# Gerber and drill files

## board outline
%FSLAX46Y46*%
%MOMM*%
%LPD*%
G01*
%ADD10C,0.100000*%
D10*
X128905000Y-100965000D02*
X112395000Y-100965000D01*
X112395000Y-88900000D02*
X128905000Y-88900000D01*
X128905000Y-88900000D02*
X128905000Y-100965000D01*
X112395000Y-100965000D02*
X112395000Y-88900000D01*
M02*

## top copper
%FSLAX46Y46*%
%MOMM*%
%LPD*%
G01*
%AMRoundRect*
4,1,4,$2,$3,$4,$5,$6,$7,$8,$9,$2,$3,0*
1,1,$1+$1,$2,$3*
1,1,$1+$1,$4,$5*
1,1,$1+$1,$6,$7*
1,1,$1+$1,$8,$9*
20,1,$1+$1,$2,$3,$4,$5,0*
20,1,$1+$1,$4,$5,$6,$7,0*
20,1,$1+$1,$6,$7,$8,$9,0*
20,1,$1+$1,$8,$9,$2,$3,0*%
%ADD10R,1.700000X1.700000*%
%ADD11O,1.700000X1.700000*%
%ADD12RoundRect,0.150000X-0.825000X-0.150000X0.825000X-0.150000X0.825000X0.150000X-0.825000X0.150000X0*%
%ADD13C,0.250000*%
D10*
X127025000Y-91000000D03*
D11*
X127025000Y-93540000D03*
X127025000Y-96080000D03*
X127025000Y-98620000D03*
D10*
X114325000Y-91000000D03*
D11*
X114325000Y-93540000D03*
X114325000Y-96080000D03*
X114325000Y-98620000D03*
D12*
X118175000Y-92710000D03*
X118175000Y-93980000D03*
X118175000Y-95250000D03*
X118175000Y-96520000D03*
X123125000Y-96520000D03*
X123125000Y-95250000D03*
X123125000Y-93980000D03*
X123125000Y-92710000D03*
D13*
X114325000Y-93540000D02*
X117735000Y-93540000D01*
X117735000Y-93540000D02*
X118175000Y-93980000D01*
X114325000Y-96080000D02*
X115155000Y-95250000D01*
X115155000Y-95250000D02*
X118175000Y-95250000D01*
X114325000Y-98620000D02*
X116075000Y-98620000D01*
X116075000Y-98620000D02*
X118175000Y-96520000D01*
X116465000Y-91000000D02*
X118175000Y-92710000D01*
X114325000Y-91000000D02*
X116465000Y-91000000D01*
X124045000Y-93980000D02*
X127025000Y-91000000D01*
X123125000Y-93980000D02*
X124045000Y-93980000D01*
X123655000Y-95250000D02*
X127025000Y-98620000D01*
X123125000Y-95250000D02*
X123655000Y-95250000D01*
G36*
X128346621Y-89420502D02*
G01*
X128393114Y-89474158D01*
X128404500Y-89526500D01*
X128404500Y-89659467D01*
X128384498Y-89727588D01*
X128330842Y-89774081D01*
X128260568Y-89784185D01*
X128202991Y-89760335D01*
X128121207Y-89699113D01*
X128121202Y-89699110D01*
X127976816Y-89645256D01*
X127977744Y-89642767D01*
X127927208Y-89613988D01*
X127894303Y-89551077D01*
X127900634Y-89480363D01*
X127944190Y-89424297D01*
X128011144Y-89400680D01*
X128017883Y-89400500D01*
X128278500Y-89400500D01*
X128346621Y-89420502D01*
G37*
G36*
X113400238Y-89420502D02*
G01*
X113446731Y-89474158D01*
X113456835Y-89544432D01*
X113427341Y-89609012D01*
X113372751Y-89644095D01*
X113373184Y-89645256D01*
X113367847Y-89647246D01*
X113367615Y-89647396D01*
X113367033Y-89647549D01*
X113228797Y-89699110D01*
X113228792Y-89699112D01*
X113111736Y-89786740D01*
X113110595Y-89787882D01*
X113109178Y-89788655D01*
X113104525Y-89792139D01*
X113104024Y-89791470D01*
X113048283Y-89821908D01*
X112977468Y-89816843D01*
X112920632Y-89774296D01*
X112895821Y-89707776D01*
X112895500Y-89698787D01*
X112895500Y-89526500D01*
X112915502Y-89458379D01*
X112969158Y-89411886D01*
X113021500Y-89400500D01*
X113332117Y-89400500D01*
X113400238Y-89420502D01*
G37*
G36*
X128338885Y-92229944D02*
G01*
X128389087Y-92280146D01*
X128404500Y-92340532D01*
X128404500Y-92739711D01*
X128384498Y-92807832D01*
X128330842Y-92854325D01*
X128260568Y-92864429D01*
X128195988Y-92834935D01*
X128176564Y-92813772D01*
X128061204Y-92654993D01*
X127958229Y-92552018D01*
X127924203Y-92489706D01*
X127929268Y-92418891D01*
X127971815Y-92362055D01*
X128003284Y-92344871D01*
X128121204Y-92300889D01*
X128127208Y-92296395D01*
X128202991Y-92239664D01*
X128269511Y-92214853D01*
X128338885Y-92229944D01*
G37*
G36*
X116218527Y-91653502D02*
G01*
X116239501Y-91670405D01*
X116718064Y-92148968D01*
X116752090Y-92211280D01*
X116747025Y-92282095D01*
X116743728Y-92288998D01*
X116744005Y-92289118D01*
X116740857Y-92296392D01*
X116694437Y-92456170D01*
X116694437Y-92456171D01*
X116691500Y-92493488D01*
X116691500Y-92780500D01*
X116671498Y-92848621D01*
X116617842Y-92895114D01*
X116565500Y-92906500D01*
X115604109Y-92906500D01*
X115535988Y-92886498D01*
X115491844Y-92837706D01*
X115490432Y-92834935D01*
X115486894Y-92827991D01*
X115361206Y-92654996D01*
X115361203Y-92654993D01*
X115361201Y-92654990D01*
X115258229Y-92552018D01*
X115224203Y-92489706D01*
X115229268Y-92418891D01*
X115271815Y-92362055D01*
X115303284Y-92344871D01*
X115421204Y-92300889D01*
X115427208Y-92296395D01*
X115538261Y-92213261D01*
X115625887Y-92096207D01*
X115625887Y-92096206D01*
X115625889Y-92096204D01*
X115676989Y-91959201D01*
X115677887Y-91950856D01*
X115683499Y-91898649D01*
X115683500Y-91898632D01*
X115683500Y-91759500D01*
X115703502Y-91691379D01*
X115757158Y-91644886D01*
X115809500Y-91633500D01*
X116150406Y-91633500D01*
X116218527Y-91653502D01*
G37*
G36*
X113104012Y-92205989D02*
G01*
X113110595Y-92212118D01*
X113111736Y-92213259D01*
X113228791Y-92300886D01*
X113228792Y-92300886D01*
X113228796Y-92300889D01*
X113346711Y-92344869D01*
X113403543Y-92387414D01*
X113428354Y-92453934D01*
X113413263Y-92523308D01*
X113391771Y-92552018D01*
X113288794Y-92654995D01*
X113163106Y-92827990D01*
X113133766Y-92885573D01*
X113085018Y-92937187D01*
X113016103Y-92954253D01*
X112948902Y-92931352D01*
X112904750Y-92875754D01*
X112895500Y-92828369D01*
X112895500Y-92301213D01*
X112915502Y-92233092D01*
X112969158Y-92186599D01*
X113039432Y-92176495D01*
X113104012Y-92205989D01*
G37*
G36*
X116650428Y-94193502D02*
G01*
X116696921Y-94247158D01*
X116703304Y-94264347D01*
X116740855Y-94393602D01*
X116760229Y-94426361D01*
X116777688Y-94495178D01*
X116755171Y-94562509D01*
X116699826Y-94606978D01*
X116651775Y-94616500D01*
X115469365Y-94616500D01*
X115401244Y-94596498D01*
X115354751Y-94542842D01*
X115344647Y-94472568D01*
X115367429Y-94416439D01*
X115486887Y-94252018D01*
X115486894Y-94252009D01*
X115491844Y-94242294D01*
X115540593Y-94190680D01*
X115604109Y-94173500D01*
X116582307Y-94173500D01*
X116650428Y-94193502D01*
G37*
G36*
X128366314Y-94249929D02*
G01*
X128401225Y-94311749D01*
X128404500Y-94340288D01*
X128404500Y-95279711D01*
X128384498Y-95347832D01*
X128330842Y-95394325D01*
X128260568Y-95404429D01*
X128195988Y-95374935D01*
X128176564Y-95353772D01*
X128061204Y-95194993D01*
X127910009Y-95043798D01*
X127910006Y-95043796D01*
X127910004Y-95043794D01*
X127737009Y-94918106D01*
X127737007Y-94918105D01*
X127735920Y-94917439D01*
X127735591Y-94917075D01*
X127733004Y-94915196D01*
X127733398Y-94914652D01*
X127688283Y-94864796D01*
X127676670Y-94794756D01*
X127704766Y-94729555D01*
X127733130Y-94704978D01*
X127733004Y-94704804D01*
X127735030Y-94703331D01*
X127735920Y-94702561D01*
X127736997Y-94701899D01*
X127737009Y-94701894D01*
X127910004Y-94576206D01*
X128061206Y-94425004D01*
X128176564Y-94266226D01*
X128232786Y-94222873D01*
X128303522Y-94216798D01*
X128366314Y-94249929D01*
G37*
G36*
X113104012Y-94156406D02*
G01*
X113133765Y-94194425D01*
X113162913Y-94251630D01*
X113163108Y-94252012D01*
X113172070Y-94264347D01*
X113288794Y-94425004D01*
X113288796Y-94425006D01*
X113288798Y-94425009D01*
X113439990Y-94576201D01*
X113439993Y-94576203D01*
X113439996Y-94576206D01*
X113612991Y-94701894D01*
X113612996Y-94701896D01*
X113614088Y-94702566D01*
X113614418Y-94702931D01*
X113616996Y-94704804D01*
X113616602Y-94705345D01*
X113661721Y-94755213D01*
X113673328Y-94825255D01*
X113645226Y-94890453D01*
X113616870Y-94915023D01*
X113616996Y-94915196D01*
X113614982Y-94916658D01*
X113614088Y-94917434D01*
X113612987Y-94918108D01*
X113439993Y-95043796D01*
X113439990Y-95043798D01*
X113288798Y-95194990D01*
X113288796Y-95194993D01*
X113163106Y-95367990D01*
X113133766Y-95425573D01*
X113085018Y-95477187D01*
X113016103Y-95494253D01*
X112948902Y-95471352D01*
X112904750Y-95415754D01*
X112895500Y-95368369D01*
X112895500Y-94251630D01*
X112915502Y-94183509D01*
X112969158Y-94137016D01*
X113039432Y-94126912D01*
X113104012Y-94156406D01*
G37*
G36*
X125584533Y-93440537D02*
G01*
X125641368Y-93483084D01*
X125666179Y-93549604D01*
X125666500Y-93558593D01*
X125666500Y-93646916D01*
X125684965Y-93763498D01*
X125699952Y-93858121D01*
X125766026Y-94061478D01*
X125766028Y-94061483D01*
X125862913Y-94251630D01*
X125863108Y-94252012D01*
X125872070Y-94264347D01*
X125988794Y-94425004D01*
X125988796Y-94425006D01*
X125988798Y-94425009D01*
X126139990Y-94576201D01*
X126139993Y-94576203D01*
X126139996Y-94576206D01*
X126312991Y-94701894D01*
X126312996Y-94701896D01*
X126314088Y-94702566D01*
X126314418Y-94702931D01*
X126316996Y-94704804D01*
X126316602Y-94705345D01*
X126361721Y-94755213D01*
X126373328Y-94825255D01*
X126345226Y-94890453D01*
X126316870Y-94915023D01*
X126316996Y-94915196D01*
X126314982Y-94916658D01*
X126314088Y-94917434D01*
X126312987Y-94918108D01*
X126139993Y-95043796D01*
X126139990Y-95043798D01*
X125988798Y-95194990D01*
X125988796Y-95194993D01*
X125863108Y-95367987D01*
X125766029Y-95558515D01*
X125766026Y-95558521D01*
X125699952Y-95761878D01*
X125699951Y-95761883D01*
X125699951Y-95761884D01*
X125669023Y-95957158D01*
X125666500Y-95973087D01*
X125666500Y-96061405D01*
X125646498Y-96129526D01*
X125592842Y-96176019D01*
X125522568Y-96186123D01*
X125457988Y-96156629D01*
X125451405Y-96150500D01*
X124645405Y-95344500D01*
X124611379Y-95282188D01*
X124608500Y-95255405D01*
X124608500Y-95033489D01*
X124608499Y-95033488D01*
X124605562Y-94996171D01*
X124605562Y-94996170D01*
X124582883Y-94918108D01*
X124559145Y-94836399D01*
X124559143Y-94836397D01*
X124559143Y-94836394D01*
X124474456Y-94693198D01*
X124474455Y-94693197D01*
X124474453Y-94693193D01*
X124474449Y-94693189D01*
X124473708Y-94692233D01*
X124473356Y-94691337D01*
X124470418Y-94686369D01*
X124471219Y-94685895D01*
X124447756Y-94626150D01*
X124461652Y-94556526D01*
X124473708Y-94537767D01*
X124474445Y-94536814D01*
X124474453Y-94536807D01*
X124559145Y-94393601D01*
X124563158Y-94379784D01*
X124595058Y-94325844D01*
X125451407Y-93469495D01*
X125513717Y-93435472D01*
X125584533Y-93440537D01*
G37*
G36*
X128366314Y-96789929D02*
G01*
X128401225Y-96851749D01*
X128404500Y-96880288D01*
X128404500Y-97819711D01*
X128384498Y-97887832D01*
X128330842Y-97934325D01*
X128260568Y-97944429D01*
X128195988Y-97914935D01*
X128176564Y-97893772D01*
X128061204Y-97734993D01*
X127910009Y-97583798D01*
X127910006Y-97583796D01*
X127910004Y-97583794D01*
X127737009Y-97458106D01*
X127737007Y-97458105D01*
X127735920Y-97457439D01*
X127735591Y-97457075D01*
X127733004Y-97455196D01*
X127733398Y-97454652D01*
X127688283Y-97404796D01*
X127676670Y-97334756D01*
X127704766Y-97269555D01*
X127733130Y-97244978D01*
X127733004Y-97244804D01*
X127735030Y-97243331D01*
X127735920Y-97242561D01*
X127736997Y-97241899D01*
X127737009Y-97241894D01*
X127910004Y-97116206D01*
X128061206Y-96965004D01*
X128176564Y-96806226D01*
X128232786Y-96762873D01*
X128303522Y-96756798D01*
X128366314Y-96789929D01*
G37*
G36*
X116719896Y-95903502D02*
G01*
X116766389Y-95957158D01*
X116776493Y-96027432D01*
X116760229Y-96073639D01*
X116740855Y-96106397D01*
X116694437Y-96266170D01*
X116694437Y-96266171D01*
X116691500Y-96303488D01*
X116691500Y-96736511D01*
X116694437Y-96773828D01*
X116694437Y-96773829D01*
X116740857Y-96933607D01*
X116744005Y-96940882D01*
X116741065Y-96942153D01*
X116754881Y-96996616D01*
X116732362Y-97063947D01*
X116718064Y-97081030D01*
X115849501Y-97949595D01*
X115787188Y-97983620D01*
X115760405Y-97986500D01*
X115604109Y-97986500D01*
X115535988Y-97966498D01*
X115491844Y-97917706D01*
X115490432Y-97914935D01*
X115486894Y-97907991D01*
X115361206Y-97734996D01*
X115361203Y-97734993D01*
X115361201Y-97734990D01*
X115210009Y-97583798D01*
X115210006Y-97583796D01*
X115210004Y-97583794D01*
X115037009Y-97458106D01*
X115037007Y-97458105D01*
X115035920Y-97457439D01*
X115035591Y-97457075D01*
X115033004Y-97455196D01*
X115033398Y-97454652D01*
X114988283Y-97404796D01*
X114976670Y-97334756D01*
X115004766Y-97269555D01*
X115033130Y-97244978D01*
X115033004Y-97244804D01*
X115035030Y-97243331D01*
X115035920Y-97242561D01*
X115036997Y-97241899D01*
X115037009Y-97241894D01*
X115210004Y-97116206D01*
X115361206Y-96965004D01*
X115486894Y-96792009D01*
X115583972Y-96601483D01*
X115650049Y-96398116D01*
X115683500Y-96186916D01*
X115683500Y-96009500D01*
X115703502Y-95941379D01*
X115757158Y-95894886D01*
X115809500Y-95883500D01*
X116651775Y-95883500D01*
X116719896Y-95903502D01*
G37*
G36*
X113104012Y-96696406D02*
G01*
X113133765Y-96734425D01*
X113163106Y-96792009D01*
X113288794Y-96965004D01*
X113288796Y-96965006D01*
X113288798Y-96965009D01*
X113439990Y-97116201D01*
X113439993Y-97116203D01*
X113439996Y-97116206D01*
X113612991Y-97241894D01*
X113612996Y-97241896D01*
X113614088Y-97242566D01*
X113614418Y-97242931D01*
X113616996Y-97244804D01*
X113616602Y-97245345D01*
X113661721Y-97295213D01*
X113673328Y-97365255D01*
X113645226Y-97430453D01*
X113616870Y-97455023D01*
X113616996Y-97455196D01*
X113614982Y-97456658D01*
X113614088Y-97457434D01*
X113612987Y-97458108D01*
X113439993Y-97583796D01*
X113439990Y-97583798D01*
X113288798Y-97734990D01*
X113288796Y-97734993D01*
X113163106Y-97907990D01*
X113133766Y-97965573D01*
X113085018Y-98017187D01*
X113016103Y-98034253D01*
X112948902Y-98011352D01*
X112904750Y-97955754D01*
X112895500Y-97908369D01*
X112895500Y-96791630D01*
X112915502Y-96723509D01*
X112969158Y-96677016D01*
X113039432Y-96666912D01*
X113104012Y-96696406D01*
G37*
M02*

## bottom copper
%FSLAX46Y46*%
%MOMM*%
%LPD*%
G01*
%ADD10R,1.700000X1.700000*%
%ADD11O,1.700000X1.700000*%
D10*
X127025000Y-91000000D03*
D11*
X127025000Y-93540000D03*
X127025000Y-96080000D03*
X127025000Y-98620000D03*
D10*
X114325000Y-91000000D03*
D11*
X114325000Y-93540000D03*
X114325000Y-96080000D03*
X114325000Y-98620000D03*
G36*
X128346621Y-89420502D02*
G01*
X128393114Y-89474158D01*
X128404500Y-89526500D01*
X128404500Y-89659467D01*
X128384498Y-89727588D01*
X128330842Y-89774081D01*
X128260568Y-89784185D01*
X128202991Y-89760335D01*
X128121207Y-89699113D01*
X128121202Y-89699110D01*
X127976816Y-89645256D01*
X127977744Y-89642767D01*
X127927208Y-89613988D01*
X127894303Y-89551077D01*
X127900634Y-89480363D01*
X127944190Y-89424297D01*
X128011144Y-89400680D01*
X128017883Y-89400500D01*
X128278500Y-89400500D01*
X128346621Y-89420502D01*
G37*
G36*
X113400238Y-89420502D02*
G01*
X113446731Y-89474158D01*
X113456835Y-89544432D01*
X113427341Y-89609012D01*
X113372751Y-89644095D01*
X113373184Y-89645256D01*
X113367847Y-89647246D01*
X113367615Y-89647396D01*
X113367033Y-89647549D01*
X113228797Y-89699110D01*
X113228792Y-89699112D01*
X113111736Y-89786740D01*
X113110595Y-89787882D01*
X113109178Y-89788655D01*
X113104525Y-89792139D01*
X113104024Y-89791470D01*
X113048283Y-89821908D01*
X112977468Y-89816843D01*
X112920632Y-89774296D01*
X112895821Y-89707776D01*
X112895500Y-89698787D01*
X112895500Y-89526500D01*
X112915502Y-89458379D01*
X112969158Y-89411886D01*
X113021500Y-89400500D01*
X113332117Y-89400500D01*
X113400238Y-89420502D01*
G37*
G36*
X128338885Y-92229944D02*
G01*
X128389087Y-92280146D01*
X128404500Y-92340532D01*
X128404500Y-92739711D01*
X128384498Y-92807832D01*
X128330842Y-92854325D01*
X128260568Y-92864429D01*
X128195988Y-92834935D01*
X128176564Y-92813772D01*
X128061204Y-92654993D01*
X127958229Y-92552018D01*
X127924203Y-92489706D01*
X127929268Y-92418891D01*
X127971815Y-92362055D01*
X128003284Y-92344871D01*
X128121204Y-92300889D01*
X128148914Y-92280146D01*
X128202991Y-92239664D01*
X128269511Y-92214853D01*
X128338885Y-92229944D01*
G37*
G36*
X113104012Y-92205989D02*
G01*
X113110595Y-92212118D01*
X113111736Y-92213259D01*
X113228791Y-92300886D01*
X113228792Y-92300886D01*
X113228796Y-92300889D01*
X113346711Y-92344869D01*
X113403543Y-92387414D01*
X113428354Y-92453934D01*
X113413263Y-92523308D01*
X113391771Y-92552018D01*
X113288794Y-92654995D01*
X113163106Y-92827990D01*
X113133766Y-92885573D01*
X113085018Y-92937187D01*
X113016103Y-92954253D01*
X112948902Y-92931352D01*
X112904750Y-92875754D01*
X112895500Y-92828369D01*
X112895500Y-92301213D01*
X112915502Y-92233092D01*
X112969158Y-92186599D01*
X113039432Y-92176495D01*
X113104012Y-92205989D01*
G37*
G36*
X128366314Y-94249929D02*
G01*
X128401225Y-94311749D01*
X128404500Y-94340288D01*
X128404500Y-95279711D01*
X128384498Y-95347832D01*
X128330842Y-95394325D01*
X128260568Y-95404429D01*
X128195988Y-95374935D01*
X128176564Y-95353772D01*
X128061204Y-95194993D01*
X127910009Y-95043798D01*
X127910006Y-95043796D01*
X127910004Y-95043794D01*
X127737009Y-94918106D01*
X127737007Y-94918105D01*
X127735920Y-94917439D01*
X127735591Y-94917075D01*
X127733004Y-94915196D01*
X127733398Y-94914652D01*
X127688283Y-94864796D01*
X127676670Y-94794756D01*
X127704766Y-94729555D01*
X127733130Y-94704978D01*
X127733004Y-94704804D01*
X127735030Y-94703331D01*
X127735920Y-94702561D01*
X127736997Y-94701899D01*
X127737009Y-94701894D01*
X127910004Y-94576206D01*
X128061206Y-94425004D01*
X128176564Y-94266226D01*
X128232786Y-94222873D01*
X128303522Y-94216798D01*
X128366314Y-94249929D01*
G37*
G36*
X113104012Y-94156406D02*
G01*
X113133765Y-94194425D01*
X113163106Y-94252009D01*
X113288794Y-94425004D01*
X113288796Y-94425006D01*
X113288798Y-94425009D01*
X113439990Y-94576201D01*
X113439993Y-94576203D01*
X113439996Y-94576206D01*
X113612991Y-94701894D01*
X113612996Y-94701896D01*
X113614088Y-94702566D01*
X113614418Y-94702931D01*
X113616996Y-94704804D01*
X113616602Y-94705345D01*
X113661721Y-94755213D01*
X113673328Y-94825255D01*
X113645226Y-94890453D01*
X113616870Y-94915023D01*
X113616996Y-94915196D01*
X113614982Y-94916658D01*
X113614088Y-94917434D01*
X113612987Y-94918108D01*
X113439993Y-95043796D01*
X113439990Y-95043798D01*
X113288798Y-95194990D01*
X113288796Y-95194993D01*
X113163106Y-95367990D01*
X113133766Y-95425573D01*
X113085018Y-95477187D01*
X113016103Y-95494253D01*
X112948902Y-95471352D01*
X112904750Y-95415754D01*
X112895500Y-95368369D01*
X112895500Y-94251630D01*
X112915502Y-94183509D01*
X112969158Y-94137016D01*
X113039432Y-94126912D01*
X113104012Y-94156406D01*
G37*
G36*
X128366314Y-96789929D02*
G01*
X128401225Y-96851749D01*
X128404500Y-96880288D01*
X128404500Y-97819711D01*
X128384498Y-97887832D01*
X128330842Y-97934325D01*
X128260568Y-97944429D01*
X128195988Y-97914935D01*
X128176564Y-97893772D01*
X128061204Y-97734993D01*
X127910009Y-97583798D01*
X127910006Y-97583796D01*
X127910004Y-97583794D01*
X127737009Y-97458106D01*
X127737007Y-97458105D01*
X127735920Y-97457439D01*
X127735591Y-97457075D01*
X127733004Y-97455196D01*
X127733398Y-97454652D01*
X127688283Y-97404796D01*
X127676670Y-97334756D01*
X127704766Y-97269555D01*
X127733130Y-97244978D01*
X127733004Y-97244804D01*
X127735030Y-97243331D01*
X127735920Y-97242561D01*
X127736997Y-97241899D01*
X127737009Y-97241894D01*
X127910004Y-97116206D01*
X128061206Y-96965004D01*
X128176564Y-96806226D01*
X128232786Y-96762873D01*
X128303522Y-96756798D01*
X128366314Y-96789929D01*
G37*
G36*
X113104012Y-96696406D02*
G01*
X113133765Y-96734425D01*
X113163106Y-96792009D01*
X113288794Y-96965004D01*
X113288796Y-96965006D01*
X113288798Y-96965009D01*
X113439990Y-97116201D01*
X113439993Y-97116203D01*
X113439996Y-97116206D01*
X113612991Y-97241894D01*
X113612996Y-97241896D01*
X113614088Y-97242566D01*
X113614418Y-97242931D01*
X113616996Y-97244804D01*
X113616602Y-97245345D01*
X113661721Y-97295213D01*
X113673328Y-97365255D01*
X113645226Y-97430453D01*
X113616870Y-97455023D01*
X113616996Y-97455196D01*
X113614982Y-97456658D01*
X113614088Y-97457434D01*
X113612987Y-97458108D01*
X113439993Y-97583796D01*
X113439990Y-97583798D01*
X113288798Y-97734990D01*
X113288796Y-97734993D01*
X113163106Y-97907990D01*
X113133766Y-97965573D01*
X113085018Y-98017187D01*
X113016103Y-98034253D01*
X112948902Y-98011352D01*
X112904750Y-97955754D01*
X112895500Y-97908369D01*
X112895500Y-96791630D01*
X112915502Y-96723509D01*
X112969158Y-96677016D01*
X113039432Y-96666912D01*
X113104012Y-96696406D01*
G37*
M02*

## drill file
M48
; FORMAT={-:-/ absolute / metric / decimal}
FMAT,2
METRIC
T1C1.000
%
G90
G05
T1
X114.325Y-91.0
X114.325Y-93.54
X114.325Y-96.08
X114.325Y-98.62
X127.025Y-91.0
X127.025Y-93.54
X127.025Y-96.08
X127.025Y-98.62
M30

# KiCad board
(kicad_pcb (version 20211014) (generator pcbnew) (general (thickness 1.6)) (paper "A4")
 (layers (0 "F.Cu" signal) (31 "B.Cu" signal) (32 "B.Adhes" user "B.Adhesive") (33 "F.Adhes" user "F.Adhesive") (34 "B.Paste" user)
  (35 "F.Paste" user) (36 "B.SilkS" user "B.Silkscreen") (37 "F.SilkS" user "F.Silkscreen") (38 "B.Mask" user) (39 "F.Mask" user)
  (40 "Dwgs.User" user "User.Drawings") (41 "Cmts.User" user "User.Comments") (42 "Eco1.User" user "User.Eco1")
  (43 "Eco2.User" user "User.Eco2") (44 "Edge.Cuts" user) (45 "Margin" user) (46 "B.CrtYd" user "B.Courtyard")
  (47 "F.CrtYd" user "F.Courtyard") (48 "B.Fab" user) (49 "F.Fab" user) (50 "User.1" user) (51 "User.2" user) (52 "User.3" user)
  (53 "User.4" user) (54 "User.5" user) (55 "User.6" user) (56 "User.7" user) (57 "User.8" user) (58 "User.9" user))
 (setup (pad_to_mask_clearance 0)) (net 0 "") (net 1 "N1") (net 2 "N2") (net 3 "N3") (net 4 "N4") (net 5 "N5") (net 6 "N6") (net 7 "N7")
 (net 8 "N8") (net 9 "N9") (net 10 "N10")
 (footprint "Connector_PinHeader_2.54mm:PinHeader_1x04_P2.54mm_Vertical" (layer "F.Cu") (at 127.025 91)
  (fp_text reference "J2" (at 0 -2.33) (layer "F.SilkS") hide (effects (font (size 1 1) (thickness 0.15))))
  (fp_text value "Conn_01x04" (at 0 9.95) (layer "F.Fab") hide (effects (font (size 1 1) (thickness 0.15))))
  (pad "1" thru_hole rect (at 0 0) (size 1.7 1.7) (drill 1) (layers *.Cu *.Mask) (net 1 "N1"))
  (pad "2" thru_hole oval (at 0 2.54) (size 1.7 1.7) (drill 1) (layers *.Cu *.Mask) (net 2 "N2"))
  (pad "3" thru_hole oval (at 0 5.08) (size 1.7 1.7) (drill 1) (layers *.Cu *.Mask) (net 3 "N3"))
  (pad "4" thru_hole oval (at 0 7.62) (size 1.7 1.7) (drill 1) (layers *.Cu *.Mask) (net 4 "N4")))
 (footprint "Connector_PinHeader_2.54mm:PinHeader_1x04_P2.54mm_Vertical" (layer "F.Cu") (at 114.325 91)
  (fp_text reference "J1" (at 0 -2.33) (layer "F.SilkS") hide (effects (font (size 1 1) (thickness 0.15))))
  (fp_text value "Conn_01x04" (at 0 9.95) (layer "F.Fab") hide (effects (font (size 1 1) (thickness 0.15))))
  (pad "1" thru_hole rect (at 0 0) (size 1.7 1.7) (drill 1) (layers *.Cu *.Mask) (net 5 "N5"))
  (pad "2" thru_hole oval (at 0 2.54) (size 1.7 1.7) (drill 1) (layers *.Cu *.Mask) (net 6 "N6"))
  (pad "3" thru_hole oval (at 0 5.08) (size 1.7 1.7) (drill 1) (layers *.Cu *.Mask) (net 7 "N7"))
  (pad "4" thru_hole oval (at 0 7.62) (size 1.7 1.7) (drill 1) (layers *.Cu *.Mask) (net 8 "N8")))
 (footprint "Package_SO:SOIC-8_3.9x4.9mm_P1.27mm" (layer "F.Cu") (at 120.65 94.615)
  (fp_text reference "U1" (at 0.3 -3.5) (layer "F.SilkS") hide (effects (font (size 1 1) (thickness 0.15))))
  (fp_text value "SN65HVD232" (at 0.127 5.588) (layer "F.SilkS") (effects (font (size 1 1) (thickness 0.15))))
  (pad "1" smd roundrect (at -2.475 -1.905) (size 1.95 0.6) (layers "F.Cu" "F.Paste" "F.Mask") (roundrect_rratio 0.25) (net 5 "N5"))
  (pad "2" smd roundrect (at -2.475 -0.635) (size 1.95 0.6) (layers "F.Cu" "F.Paste" "F.Mask") (roundrect_rratio 0.25) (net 6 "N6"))
  (pad "3" smd roundrect (at -2.475 0.635) (size 1.95 0.6) (layers "F.Cu" "F.Paste" "F.Mask") (roundrect_rratio 0.25) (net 7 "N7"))
  (pad "4" smd roundrect (at -2.475 1.905) (size 1.95 0.6) (layers "F.Cu" "F.Paste" "F.Mask") (roundrect_rratio 0.25) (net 8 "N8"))
  (pad "5" smd roundrect (at 2.475 1.905) (size 1.95 0.6) (layers "F.Cu" "F.Paste" "F.Mask") (roundrect_rratio 0.25) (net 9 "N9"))
  (pad "6" smd roundrect (at 2.475 0.635) (size 1.95 0.6) (layers "F.Cu" "F.Paste" "F.Mask") (roundrect_rratio 0.25) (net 4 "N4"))
  (pad "7" smd roundrect (at 2.475 -0.635) (size 1.95 0.6) (layers "F.Cu" "F.Paste" "F.Mask") (roundrect_rratio 0.25) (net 1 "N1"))
  (pad "8" smd roundrect (at 2.475 -1.905) (size 1.95 0.6) (layers "F.Cu" "F.Paste" "F.Mask") (roundrect_rratio 0.25) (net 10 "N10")))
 (gr_line (start 128.905 100.965) (end 112.395 100.965) (layer "Edge.Cuts") (width 0.1))
 (gr_line (start 112.395 88.9) (end 128.905 88.9) (layer "Edge.Cuts") (width 0.1))
 (gr_line (start 128.905 88.9) (end 128.905 100.965) (layer "Edge.Cuts") (width 0.1))
 (gr_line (start 112.395 100.965) (end 112.395 88.9) (layer "Edge.Cuts") (width 0.1))
 (segment (start 114.325 93.54) (end 117.735 93.54) (width 0.25) (layer "F.Cu") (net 6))
 (segment (start 117.735 93.54) (end 118.175 93.98) (width 0.25) (layer "F.Cu") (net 6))
 (segment (start 114.325 96.08) (end 115.155 95.25) (width 0.25) (layer "F.Cu") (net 7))
 (segment (start 115.155 95.25) (end 118.175 95.25) (width 0.25) (layer "F.Cu") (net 7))
 (segment (start 114.325 98.62) (end 116.075 98.62) (width 0.25) (layer "F.Cu") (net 8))
 (segment (start 116.075 98.62) (end 118.175 96.52) (width 0.25) (layer "F.Cu") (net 8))
 (segment (start 116.465 91) (end 118.175 92.71) (width 0.25) (layer "F.Cu") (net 5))
 (segment (start 114.325 91) (end 116.465 91) (width 0.25) (layer "F.Cu") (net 5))
 (segment (start 124.045 93.98) (end 127.025 91) (width 0.25) (layer "F.Cu") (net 1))
 (segment (start 123.125 93.98) (end 124.045 93.98) (width 0.25) (layer "F.Cu") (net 1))
 (segment (start 123.655 95.25) (end 127.025 98.62) (width 0.25) (layer "F.Cu") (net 4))
 (segment (start 123.125 95.25) (end 123.655 95.25) (width 0.25) (layer "F.Cu") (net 4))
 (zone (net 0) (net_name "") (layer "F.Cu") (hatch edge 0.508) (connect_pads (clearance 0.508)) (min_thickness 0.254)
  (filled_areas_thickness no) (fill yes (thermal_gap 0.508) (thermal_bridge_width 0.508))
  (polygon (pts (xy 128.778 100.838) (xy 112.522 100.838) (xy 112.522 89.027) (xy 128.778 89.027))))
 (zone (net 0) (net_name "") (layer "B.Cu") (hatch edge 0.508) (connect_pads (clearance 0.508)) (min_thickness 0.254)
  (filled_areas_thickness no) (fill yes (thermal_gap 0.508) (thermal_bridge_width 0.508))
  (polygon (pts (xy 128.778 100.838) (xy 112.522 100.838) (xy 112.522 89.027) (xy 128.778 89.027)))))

